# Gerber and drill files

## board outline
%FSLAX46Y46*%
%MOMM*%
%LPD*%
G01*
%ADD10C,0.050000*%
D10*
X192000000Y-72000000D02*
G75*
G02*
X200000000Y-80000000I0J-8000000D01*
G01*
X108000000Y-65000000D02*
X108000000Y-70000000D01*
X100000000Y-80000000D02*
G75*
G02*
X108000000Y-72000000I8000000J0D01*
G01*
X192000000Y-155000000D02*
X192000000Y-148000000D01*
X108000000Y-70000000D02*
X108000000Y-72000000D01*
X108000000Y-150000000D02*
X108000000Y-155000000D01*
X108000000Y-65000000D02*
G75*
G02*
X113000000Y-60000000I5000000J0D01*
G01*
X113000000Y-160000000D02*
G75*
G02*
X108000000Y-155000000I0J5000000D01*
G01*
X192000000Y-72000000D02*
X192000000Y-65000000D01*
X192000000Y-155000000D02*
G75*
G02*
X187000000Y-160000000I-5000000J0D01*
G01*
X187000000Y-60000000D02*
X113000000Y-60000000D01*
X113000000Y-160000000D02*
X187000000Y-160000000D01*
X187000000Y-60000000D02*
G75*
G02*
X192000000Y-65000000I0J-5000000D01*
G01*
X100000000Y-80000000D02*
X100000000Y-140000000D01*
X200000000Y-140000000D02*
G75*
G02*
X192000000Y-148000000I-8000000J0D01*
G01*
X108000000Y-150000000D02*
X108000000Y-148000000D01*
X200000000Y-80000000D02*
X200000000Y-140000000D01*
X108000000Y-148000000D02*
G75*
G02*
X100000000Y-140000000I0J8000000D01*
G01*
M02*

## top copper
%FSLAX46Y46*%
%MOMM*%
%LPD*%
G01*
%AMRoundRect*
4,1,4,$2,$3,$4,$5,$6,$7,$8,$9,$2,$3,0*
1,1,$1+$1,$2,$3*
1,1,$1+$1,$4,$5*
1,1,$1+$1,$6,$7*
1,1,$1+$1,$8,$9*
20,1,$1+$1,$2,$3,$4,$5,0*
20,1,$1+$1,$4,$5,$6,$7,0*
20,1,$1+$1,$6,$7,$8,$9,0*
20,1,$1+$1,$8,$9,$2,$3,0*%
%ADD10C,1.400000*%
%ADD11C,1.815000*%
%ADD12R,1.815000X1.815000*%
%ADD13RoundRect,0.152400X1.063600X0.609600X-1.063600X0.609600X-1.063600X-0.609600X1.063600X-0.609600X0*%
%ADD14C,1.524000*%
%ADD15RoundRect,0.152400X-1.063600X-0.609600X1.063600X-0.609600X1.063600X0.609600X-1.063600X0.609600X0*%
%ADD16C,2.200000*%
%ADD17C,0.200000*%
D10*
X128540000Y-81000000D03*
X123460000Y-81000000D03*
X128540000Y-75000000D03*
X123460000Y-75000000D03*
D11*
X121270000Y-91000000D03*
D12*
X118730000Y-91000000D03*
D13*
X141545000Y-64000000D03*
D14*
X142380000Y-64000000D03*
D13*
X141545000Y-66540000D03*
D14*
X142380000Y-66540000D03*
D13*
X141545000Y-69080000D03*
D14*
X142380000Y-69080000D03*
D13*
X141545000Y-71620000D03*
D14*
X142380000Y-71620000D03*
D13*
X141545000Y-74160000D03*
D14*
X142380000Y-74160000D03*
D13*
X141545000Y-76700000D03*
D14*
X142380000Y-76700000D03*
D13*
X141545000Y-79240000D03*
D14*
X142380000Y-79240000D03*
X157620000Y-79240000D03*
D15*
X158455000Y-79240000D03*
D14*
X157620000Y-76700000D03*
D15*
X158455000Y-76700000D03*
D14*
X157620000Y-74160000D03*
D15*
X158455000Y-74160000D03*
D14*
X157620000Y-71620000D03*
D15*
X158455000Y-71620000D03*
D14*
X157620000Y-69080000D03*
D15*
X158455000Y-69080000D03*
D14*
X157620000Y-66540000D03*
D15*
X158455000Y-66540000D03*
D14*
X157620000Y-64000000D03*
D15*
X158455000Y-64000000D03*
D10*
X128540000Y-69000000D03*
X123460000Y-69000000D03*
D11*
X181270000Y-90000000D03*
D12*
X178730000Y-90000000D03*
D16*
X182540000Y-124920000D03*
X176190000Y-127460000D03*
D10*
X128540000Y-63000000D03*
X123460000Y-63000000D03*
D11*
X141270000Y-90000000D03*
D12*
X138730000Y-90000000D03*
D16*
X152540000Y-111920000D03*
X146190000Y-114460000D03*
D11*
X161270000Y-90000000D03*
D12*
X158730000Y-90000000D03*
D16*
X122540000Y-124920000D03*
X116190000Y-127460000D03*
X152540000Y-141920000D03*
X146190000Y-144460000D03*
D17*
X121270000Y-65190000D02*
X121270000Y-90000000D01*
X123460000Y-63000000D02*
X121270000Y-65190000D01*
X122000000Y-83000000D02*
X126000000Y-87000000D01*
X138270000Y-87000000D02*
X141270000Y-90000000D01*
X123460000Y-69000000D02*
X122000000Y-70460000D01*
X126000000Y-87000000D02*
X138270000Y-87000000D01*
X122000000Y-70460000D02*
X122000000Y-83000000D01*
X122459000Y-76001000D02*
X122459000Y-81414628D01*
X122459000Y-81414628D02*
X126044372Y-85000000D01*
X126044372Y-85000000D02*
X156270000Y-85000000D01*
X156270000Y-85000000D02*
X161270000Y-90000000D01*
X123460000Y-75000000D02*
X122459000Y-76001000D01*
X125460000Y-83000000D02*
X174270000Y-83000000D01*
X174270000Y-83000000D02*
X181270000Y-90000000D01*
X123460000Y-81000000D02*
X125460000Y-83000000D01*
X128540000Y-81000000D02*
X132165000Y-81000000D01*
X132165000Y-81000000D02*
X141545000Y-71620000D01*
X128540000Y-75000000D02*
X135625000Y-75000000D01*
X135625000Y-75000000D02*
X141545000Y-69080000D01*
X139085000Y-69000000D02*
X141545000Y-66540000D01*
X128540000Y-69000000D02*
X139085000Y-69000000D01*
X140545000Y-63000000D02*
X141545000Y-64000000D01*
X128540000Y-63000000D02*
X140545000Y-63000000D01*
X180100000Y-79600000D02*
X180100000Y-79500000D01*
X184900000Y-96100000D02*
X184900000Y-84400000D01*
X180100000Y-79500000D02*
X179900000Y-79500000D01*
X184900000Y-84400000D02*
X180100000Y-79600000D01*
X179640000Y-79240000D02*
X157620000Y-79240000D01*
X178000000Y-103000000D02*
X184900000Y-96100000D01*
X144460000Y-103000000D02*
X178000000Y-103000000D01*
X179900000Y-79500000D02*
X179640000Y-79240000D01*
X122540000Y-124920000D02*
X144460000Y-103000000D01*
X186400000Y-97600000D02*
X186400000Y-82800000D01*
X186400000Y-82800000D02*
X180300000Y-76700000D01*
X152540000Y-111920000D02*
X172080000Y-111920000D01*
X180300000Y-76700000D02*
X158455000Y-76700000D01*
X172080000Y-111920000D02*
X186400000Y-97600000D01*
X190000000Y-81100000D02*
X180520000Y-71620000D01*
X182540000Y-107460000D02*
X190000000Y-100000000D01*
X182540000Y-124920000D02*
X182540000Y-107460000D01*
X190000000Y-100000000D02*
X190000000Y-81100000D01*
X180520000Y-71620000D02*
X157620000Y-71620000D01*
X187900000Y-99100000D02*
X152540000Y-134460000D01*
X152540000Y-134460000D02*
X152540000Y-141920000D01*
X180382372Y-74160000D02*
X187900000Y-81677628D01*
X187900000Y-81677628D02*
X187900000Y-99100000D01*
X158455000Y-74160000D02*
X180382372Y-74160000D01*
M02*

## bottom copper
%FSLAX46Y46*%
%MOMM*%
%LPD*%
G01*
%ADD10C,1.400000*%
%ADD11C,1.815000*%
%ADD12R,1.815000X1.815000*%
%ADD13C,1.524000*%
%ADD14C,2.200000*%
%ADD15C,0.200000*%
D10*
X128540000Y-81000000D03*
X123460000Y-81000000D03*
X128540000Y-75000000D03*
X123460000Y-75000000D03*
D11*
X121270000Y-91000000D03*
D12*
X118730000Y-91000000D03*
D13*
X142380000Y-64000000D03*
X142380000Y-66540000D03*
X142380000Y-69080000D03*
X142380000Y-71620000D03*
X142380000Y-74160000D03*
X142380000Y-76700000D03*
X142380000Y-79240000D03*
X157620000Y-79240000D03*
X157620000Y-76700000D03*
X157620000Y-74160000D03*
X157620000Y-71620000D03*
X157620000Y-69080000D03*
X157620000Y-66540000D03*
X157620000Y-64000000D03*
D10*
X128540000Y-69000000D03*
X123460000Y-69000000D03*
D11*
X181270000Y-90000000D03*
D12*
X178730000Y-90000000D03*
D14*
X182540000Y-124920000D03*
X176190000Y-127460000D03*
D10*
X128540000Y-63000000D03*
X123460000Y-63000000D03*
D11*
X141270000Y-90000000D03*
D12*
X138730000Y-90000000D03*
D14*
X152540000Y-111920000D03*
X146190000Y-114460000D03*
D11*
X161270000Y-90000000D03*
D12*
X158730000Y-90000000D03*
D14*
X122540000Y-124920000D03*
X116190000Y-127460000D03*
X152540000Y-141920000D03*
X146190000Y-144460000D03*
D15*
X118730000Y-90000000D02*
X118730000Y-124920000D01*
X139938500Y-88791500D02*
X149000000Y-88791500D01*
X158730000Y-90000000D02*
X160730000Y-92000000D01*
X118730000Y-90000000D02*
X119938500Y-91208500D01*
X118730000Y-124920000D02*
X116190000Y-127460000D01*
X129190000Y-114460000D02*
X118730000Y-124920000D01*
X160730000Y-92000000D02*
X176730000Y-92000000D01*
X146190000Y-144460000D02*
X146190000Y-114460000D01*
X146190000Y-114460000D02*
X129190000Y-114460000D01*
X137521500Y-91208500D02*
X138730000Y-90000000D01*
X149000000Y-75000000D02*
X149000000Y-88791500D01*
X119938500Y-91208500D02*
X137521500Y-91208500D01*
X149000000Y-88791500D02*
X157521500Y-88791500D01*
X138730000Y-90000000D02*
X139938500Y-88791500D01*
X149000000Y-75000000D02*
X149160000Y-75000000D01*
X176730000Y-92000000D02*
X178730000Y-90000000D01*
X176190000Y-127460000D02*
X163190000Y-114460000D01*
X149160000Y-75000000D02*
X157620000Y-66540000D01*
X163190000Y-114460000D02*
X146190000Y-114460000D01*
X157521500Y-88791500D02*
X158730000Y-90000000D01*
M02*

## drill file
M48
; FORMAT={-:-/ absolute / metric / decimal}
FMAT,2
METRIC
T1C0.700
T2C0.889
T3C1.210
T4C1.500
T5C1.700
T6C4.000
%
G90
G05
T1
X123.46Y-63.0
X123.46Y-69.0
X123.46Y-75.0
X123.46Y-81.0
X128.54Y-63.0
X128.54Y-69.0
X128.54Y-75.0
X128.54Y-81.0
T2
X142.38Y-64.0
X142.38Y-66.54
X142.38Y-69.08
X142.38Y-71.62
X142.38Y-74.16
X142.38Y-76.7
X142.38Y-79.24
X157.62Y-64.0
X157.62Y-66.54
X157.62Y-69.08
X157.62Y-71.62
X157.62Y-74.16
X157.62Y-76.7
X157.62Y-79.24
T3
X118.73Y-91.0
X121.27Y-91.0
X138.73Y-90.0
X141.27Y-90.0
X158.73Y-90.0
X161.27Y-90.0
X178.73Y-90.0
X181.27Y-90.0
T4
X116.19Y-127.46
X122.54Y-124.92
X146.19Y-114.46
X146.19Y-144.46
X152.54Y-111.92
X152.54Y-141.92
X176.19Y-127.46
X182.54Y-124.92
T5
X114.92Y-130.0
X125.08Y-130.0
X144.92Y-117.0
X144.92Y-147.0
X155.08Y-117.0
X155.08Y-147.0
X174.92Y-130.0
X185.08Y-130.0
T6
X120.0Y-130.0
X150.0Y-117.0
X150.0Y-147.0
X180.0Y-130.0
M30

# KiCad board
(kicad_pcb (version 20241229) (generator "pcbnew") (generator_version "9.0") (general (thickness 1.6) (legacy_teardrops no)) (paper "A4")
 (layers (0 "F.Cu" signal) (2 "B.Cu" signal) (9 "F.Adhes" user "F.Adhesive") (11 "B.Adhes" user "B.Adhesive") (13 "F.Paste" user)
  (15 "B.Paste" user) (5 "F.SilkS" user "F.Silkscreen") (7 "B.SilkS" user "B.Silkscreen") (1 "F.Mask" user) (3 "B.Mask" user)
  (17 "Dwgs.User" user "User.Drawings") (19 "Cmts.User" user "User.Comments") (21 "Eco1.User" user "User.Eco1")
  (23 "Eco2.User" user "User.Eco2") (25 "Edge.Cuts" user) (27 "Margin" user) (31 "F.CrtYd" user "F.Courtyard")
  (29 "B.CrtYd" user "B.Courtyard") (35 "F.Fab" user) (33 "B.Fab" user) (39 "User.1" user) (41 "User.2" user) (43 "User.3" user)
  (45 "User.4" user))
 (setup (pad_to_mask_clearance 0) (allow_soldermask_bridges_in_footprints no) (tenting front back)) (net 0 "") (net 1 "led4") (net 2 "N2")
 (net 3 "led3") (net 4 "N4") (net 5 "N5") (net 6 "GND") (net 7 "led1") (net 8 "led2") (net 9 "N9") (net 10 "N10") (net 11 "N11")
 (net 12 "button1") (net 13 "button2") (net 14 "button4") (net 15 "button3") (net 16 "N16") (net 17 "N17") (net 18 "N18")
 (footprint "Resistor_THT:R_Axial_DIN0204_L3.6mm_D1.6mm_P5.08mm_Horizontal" (layer "F.Cu") (at 128.54 81 180)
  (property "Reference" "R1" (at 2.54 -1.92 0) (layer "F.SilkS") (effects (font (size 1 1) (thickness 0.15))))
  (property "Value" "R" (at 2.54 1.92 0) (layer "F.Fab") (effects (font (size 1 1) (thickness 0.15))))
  (pad "1" thru_hole circle (at 0 0 180) (size 1.4 1.4) (drill 0.7) (layers "*.Cu" "*.Mask") (remove_unused_layers no) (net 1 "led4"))
  (pad "2" thru_hole circle (at 5.08 0 180) (size 1.4 1.4) (drill 0.7) (layers "*.Cu" "*.Mask") (remove_unused_layers no) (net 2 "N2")))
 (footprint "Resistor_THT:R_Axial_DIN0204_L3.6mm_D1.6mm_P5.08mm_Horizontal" (layer "F.Cu") (at 128.54 75 180)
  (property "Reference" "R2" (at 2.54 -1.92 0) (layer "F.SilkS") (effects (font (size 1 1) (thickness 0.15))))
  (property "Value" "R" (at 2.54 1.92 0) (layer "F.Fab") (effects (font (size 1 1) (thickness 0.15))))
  (pad "1" thru_hole circle (at 0 0 180) (size 1.4 1.4) (drill 0.7) (layers "*.Cu" "*.Mask") (remove_unused_layers no) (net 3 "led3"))
  (pad "2" thru_hole circle (at 5.08 0 180) (size 1.4 1.4) (drill 0.7) (layers "*.Cu" "*.Mask") (remove_unused_layers no) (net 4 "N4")))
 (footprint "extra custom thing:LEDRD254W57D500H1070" (layer "F.Cu") (at 120 91)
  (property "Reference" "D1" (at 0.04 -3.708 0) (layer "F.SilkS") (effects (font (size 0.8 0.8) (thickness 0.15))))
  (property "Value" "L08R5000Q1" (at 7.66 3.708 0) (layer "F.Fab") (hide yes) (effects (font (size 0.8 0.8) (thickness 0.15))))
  (pad "A" thru_hole circle (at 1.27 0) (size 1.815 1.815) (drill 1.21) (layers "*.Cu" "*.Mask") (remove_unused_layers no) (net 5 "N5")
   (solder_mask_margin 0.102))
  (pad "C" thru_hole rect (at -1.27 0) (size 1.815 1.815) (drill 1.21) (layers "*.Cu" "*.Mask") (remove_unused_layers no) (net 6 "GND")
   (solder_mask_margin 0.102)))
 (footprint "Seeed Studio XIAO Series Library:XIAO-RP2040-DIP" (layer "F.Cu") (at 150 71.62)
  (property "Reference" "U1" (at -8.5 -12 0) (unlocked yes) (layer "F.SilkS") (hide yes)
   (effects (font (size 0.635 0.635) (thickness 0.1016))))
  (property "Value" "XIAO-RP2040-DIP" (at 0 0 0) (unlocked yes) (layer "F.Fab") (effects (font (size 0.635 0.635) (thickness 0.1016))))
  (pad "1" smd roundrect (at -8.455 -7.62 180) (size 2.432 1.524) (layers "F.Cu" "F.Mask") (roundrect_rratio 0.1) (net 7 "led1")
   (thermal_bridge_angle 45))
  (pad "1" thru_hole circle (at -7.62 -7.62 180) (size 1.524 1.524) (drill 0.889) (layers "*.Cu" "*.Mask") (remove_unused_layers no)
   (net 7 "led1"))
  (pad "2" smd roundrect (at -8.455 -5.08 180) (size 2.432 1.524) (layers "F.Cu" "F.Mask") (roundrect_rratio 0.1) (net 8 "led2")
   (thermal_bridge_angle 45))
  (pad "2" thru_hole circle (at -7.62 -5.08 180) (size 1.524 1.524) (drill 0.889) (layers "*.Cu" "*.Mask") (remove_unused_layers no)
   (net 8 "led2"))
  (pad "3" smd roundrect (at -8.455 -2.54 180) (size 2.432 1.524) (layers "F.Cu" "F.Mask") (roundrect_rratio 0.1) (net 3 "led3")
   (thermal_bridge_angle 45))
  (pad "3" thru_hole circle (at -7.62 -2.54 180) (size 1.524 1.524) (drill 0.889) (layers "*.Cu" "*.Mask") (remove_unused_layers no)
   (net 3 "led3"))
  (pad "4" smd roundrect (at -8.455 0 180) (size 2.432 1.524) (layers "F.Cu" "F.Mask") (roundrect_rratio 0.1) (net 1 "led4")
   (thermal_bridge_angle 45))
  (pad "4" thru_hole circle (at -7.62 0 180) (size 1.524 1.524) (drill 0.889) (layers "*.Cu" "*.Mask") (remove_unused_layers no)
   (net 1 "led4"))
  (pad "5" smd roundrect (at -8.455 2.54 180) (size 2.432 1.524) (layers "F.Cu" "F.Mask") (roundrect_rratio 0.1) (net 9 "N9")
   (thermal_bridge_angle 45))
  (pad "5" thru_hole circle (at -7.62 2.54 180) (size 1.524 1.524) (drill 0.889) (layers "*.Cu" "*.Mask") (remove_unused_layers no)
   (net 9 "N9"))
  (pad "6" smd roundrect (at -8.455 5.08 180) (size 2.432 1.524) (layers "F.Cu" "F.Mask") (roundrect_rratio 0.1) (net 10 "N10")
   (thermal_bridge_angle 45))
  (pad "6" thru_hole circle (at -7.62 5.08 180) (size 1.524 1.524) (drill 0.889) (layers "*.Cu" "*.Mask") (remove_unused_layers no)
   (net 10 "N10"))
  (pad "7" smd roundrect (at -8.455 7.62 180) (size 2.432 1.524) (layers "F.Cu" "F.Mask") (roundrect_rratio 0.1) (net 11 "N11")
   (thermal_bridge_angle 45))
  (pad "7" thru_hole circle (at -7.62 7.62 180) (size 1.524 1.524) (drill 0.889) (layers "*.Cu" "*.Mask") (remove_unused_layers no)
   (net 11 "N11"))
  (pad "8" thru_hole circle (at 7.62 7.62) (size 1.524 1.524) (drill 0.889) (layers "*.Cu" "*.Mask") (remove_unused_layers no)
   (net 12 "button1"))
  (pad "8" smd roundrect (at 8.455 7.62) (size 2.432 1.524) (layers "F.Cu" "F.Mask") (roundrect_rratio 0.1) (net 12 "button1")
   (thermal_bridge_angle 45))
  (pad "9" thru_hole circle (at 7.62 5.08) (size 1.524 1.524) (drill 0.889) (layers "*.Cu" "*.Mask") (remove_unused_layers no)
   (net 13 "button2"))
  (pad "9" smd roundrect (at 8.455 5.08) (size 2.432 1.524) (layers "F.Cu" "F.Mask") (roundrect_rratio 0.1) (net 13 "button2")
   (thermal_bridge_angle 45))
  (pad "10" thru_hole circle (at 7.62 2.54) (size 1.524 1.524) (drill 0.889) (layers "*.Cu" "*.Mask") (remove_unused_layers no)
   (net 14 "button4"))
  (pad "10" smd roundrect (at 8.455 2.54) (size 2.432 1.524) (layers "F.Cu" "F.Mask") (roundrect_rratio 0.1) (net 14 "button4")
   (thermal_bridge_angle 45))
  (pad "11" thru_hole circle (at 7.62 0) (size 1.524 1.524) (drill 0.889) (layers "*.Cu" "*.Mask") (remove_unused_layers no)
   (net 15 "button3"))
  (pad "11" smd roundrect (at 8.455 0) (size 2.432 1.524) (layers "F.Cu" "F.Mask") (roundrect_rratio 0.1) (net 15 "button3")
   (thermal_bridge_angle 45))
  (pad "12" thru_hole circle (at 7.62 -2.54) (size 1.524 1.524) (drill 0.889) (layers "*.Cu" "*.Mask") (remove_unused_layers no)
   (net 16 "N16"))
  (pad "12" smd roundrect (at 8.455 -2.54) (size 2.432 1.524) (layers "F.Cu" "F.Mask") (roundrect_rratio 0.1) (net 16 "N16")
   (thermal_bridge_angle 45))
  (pad "13" thru_hole circle (at 7.62 -5.08) (size 1.524 1.524) (drill 0.889) (layers "*.Cu" "*.Mask") (remove_unused_layers no)
   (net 6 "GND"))
  (pad "13" smd roundrect (at 8.455 -5.08) (size 2.432 1.524) (layers "F.Cu" "F.Mask") (roundrect_rratio 0.1) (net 6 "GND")
   (thermal_bridge_angle 45))
  (pad "14" thru_hole circle (at 7.62 -7.62) (size 1.524 1.524) (drill 0.889) (layers "*.Cu" "*.Mask") (remove_unused_layers no)
   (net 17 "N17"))
  (pad "14" smd roundrect (at 8.455 -7.62) (size 2.432 1.524) (layers "F.Cu" "F.Mask") (roundrect_rratio 0.1) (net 17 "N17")
   (thermal_bridge_angle 45)))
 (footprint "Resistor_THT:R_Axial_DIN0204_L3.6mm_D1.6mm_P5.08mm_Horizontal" (layer "F.Cu") (at 128.54 69 180)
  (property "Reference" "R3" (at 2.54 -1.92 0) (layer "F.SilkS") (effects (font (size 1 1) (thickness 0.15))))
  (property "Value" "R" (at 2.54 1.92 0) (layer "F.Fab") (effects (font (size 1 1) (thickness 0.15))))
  (pad "1" thru_hole circle (at 0 0 180) (size 1.4 1.4) (drill 0.7) (layers "*.Cu" "*.Mask") (remove_unused_layers no) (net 8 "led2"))
  (pad "2" thru_hole circle (at 5.08 0 180) (size 1.4 1.4) (drill 0.7) (layers "*.Cu" "*.Mask") (remove_unused_layers no) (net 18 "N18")))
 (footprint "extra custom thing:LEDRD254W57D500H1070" (layer "F.Cu") (at 180 90)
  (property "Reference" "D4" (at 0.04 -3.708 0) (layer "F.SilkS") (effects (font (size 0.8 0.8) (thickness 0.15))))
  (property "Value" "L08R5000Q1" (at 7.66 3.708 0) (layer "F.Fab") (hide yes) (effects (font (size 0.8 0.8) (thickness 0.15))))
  (pad "A" thru_hole circle (at 1.27 0) (size 1.815 1.815) (drill 1.21) (layers "*.Cu" "*.Mask") (remove_unused_layers no) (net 2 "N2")
   (solder_mask_margin 0.102))
  (pad "C" thru_hole rect (at -1.27 0) (size 1.815 1.815) (drill 1.21) (layers "*.Cu" "*.Mask") (remove_unused_layers no) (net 6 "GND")
   (solder_mask_margin 0.102)))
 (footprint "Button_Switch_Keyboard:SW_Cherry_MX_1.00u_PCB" (layer "F.Cu") (at 182.54 124.92)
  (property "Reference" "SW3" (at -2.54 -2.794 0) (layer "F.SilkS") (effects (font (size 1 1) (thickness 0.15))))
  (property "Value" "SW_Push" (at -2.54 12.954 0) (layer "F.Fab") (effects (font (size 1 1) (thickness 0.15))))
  (pad "" np_thru_hole circle (at -7.62 5.08) (size 1.7 1.7) (drill 1.7) (layers "*.Cu" "*.Mask"))
  (pad "" np_thru_hole circle (at -2.54 5.08) (size 4 4) (drill 4) (layers "*.Cu" "*.Mask"))
  (pad "" np_thru_hole circle (at 2.54 5.08) (size 1.7 1.7) (drill 1.7) (layers "*.Cu" "*.Mask"))
  (pad "1" thru_hole circle (at 0 0) (size 2.2 2.2) (drill 1.5) (layers "*.Cu" "*.Mask") (remove_unused_layers no) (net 15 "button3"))
  (pad "2" thru_hole circle (at -6.35 2.54) (size 2.2 2.2) (drill 1.5) (layers "*.Cu" "*.Mask") (remove_unused_layers no) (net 6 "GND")))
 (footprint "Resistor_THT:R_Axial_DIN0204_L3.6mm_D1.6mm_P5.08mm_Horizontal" (layer "F.Cu") (at 128.54 63 180)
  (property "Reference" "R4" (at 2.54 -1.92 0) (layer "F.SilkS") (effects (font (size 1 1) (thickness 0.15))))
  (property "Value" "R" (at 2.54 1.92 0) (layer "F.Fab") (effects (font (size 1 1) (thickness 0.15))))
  (pad "1" thru_hole circle (at 0 0 180) (size 1.4 1.4) (drill 0.7) (layers "*.Cu" "*.Mask") (remove_unused_layers no) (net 7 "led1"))
  (pad "2" thru_hole circle (at 5.08 0 180) (size 1.4 1.4) (drill 0.7) (layers "*.Cu" "*.Mask") (remove_unused_layers no) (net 5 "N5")))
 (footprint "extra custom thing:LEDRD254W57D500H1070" (layer "F.Cu") (at 140 90)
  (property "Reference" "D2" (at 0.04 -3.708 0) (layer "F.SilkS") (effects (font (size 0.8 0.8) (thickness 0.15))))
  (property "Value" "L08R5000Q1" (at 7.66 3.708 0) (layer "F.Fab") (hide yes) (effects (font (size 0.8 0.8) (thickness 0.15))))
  (pad "A" thru_hole circle (at 1.27 0) (size 1.815 1.815) (drill 1.21) (layers "*.Cu" "*.Mask") (remove_unused_layers no) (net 18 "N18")
   (solder_mask_margin 0.102))
  (pad "C" thru_hole rect (at -1.27 0) (size 1.815 1.815) (drill 1.21) (layers "*.Cu" "*.Mask") (remove_unused_layers no) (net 6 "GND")
   (solder_mask_margin 0.102)))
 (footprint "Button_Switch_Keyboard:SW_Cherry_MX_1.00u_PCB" (layer "F.Cu") (at 152.54 111.92)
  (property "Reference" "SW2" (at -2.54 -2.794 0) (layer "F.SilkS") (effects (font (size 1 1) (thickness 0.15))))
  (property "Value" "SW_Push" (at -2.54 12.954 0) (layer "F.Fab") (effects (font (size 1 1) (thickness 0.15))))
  (pad "" np_thru_hole circle (at -7.62 5.08) (size 1.7 1.7) (drill 1.7) (layers "*.Cu" "*.Mask"))
  (pad "" np_thru_hole circle (at -2.54 5.08) (size 4 4) (drill 4) (layers "*.Cu" "*.Mask"))
  (pad "" np_thru_hole circle (at 2.54 5.08) (size 1.7 1.7) (drill 1.7) (layers "*.Cu" "*.Mask"))
  (pad "1" thru_hole circle (at 0 0) (size 2.2 2.2) (drill 1.5) (layers "*.Cu" "*.Mask") (remove_unused_layers no) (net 13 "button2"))
  (pad "2" thru_hole circle (at -6.35 2.54) (size 2.2 2.2) (drill 1.5) (layers "*.Cu" "*.Mask") (remove_unused_layers no) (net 6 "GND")))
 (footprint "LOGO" (layer "F.Cu") (at 129 104)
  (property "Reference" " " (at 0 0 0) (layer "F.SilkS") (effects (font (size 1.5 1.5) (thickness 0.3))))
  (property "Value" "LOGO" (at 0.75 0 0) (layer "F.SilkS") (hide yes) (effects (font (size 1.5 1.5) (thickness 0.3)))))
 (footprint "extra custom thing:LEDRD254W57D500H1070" (layer "F.Cu") (at 160 90)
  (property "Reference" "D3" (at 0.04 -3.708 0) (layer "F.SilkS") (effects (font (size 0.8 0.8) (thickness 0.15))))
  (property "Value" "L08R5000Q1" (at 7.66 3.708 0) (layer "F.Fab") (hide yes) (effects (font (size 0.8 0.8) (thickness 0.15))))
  (pad "A" thru_hole circle (at 1.27 0) (size 1.815 1.815) (drill 1.21) (layers "*.Cu" "*.Mask") (remove_unused_layers no) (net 4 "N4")
   (solder_mask_margin 0.102))
  (pad "C" thru_hole rect (at -1.27 0) (size 1.815 1.815) (drill 1.21) (layers "*.Cu" "*.Mask") (remove_unused_layers no) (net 6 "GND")
   (solder_mask_margin 0.102)))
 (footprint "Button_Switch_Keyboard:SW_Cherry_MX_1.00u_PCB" (layer "F.Cu") (at 122.54 124.92)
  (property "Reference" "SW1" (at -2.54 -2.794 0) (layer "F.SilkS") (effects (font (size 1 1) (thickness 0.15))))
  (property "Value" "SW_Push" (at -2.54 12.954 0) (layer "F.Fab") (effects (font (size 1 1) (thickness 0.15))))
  (pad "" np_thru_hole circle (at -7.62 5.08) (size 1.7 1.7) (drill 1.7) (layers "*.Cu" "*.Mask"))
  (pad "" np_thru_hole circle (at -2.54 5.08) (size 4 4) (drill 4) (layers "*.Cu" "*.Mask"))
  (pad "" np_thru_hole circle (at 2.54 5.08) (size 1.7 1.7) (drill 1.7) (layers "*.Cu" "*.Mask"))
  (pad "1" thru_hole circle (at 0 0) (size 2.2 2.2) (drill 1.5) (layers "*.Cu" "*.Mask") (remove_unused_layers no) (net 12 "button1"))
  (pad "2" thru_hole circle (at -6.35 2.54) (size 2.2 2.2) (drill 1.5) (layers "*.Cu" "*.Mask") (remove_unused_layers no) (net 6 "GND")))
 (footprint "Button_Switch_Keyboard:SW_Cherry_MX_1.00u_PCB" (layer "F.Cu") (at 152.54 141.92)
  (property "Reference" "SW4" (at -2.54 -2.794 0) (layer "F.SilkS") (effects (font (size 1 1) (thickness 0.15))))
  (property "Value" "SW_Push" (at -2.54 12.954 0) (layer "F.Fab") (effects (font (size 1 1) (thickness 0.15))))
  (pad "" np_thru_hole circle (at -7.62 5.08) (size 1.7 1.7) (drill 1.7) (layers "*.Cu" "*.Mask"))
  (pad "" np_thru_hole circle (at -2.54 5.08) (size 4 4) (drill 4) (layers "*.Cu" "*.Mask"))
  (pad "" np_thru_hole circle (at 2.54 5.08) (size 1.7 1.7) (drill 1.7) (layers "*.Cu" "*.Mask"))
  (pad "1" thru_hole circle (at 0 0) (size 2.2 2.2) (drill 1.5) (layers "*.Cu" "*.Mask") (remove_unused_layers no) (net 14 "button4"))
  (pad "2" thru_hole circle (at -6.35 2.54) (size 2.2 2.2) (drill 1.5) (layers "*.Cu" "*.Mask") (remove_unused_layers no) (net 6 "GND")))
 (gr_arc (start 192 72) (mid 197.656854 74.343146) (end 200 80) (stroke (width 0.05) (type default)) (layer "Edge.Cuts"))
 (gr_line (start 108 65) (end 108 70) (stroke (width 0.05) (type default)) (layer "Edge.Cuts"))
 (gr_arc (start 100 80) (mid 102.343146 74.343146) (end 108 72) (stroke (width 0.05) (type default)) (layer "Edge.Cuts"))
 (gr_line (start 192 155) (end 192 148) (stroke (width 0.05) (type default)) (layer "Edge.Cuts"))
 (gr_line (start 108 70) (end 108 72) (stroke (width 0.05) (type default)) (layer "Edge.Cuts"))
 (gr_line (start 108 150) (end 108 155) (stroke (width 0.05) (type default)) (locked yes) (layer "Edge.Cuts"))
 (gr_arc (start 108 65) (mid 109.464466 61.464466) (end 113 60) (stroke (width 0.05) (type default)) (layer "Edge.Cuts"))
 (gr_arc (start 113 160) (mid 109.464466 158.535534) (end 108 155) (stroke (width 0.05) (type default)) (layer "Edge.Cuts"))
 (gr_line (start 192 72) (end 192 65) (stroke (width 0.05) (type default)) (layer "Edge.Cuts"))
 (gr_arc (start 192 155) (mid 190.535534 158.535534) (end 187 160) (stroke (width 0.05) (type default)) (layer "Edge.Cuts"))
 (gr_line (start 187 60) (end 113 60) (stroke (width 0.05) (type default)) (layer "Edge.Cuts"))
 (gr_line (start 113 160) (end 187 160) (stroke (width 0.05) (type default)) (layer "Edge.Cuts"))
 (gr_arc (start 187 60) (mid 190.535534 61.464466) (end 192 65) (stroke (width 0.05) (type default)) (layer "Edge.Cuts"))
 (gr_line (start 100 80) (end 100 140) (stroke (width 0.05) (type default)) (layer "Edge.Cuts"))
 (gr_arc (start 200 140) (mid 197.656854 145.656854) (end 192 148) (stroke (width 0.05) (type default)) (layer "Edge.Cuts"))
 (gr_line (start 108 150) (end 108 148) (stroke (width 0.05) (type default)) (layer "Edge.Cuts"))
 (gr_line (start 200 80) (end 200 140) (stroke (width 0.05) (type default)) (layer "Edge.Cuts"))
 (gr_arc (start 108 148) (mid 102.343146 145.656854) (end 100 140) (stroke (width 0.05) (type default)) (layer "Edge.Cuts"))
 (segment (start 121.27 65.19) (end 121.27 90) (width 0.2) (layer "F.Cu") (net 5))
 (segment (start 123.46 63) (end 121.27 65.19) (width 0.2) (layer "F.Cu") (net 5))
 (segment (start 118.73 90) (end 118.73 124.92) (width 0.2) (layer "B.Cu") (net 6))
 (segment (start 139.9385 88.7915) (end 149 88.7915) (width 0.2) (layer "B.Cu") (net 6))
 (segment (start 158.73 90) (end 160.73 92) (width 0.2) (layer "B.Cu") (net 6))
 (segment (start 118.73 90) (end 119.9385 91.2085) (width 0.2) (layer "B.Cu") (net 6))
 (segment (start 118.73 124.92) (end 116.19 127.46) (width 0.2) (layer "B.Cu") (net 6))
 (segment (start 129.19 114.46) (end 118.73 124.92) (width 0.2) (layer "B.Cu") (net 6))
 (segment (start 160.73 92) (end 176.73 92) (width 0.2) (layer "B.Cu") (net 6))
 (segment (start 146.19 144.46) (end 146.19 114.46) (width 0.2) (layer "B.Cu") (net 6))
 (segment (start 146.19 114.46) (end 129.19 114.46) (width 0.2) (layer "B.Cu") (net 6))
 (segment (start 137.5215 91.2085) (end 138.73 90) (width 0.2) (layer "B.Cu") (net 6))
 (segment (start 149 75) (end 149 88.7915) (width 0.2) (layer "B.Cu") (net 6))
 (segment (start 119.9385 91.2085) (end 137.5215 91.2085) (width 0.2) (layer "B.Cu") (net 6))
 (segment (start 149 88.7915) (end 157.5215 88.7915) (width 0.2) (layer "B.Cu") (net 6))
 (segment (start 138.73 90) (end 139.9385 88.7915) (width 0.2) (layer "B.Cu") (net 6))
 (segment (start 149 75) (end 149.16 75) (width 0.2) (layer "B.Cu") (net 6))
 (segment (start 176.73 92) (end 178.73 90) (width 0.2) (layer "B.Cu") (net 6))
 (segment (start 176.19 127.46) (end 163.19 114.46) (width 0.2) (layer "B.Cu") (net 6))
 (segment (start 149.16 75) (end 157.62 66.54) (width 0.2) (layer "B.Cu") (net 6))
 (segment (start 163.19 114.46) (end 146.19 114.46) (width 0.2) (layer "B.Cu") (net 6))
 (segment (start 157.5215 88.7915) (end 158.73 90) (width 0.2) (layer "B.Cu") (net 6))
 (segment (start 122 83) (end 126 87) (width 0.2) (layer "F.Cu") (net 18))
 (segment (start 138.27 87) (end 141.27 90) (width 0.2) (layer "F.Cu") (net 18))
 (segment (start 123.46 69) (end 122 70.46) (width 0.2) (layer "F.Cu") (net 18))
 (segment (start 126 87) (end 138.27 87) (width 0.2) (layer "F.Cu") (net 18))
 (segment (start 122 70.46) (end 122 83) (width 0.2) (layer "F.Cu") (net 18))
 (segment (start 122.459 76.001) (end 122.459 81.414628) (width 0.2) (layer "F.Cu") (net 4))
 (segment (start 122.459 81.414628) (end 126.044372 85) (width 0.2) (layer "F.Cu") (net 4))
 (segment (start 126.044372 85) (end 156.27 85) (width 0.2) (layer "F.Cu") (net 4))
 (segment (start 156.27 85) (end 161.27 90) (width 0.2) (layer "F.Cu") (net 4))
 (segment (start 123.46 75) (end 122.459 76.001) (width 0.2) (layer "F.Cu") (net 4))
 (segment (start 125.46 83) (end 174.27 83) (width 0.2) (layer "F.Cu") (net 2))
 (segment (start 174.27 83) (end 181.27 90) (width 0.2) (layer "F.Cu") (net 2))
 (segment (start 123.46 81) (end 125.46 83) (width 0.2) (layer "F.Cu") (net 2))
 (segment (start 128.54 81) (end 132.165 81) (width 0.2) (layer "F.Cu") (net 1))
 (segment (start 132.165 81) (end 141.545 71.62) (width 0.2) (layer "F.Cu") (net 1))
 (segment (start 128.54 75) (end 135.625 75) (width 0.2) (layer "F.Cu") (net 3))
 (segment (start 135.625 75) (end 141.545 69.08) (width 0.2) (layer "F.Cu") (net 3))
 (segment (start 139.085 69) (end 141.545 66.54) (width 0.2) (layer "F.Cu") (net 8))
 (segment (start 128.54 69) (end 139.085 69) (width 0.2) (layer "F.Cu") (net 8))
 (segment (start 140.545 63) (end 141.545 64) (width 0.2) (layer "F.Cu") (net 7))
 (segment (start 128.54 63) (end 140.545 63) (width 0.2) (layer "F.Cu") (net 7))
 (segment (start 180.1 79.6) (end 180.1 79.5) (width 0.2) (layer "F.Cu") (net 12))
 (segment (start 184.9 96.1) (end 184.9 84.4) (width 0.2) (layer "F.Cu") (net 12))
 (segment (start 180.1 79.5) (end 179.9 79.5) (width 0.2) (layer "F.Cu") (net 12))
 (segment (start 184.9 84.4) (end 180.1 79.6) (width 0.2) (layer "F.Cu") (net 12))
 (segment (start 179.64 79.24) (end 157.62 79.24) (width 0.2) (layer "F.Cu") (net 12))
 (segment (start 178 103) (end 184.9 96.1) (width 0.2) (layer "F.Cu") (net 12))
 (segment (start 144.46 103) (end 178 103) (width 0.2) (layer "F.Cu") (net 12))
 (segment (start 179.9 79.5) (end 179.64 79.24) (width 0.2) (layer "F.Cu") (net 12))
 (segment (start 122.54 124.92) (end 144.46 103) (width 0.2) (layer "F.Cu") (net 12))
 (segment (start 186.4 97.6) (end 186.4 82.8) (width 0.2) (layer "F.Cu") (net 13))
 (segment (start 186.4 82.8) (end 180.3 76.7) (width 0.2) (layer "F.Cu") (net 13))
 (segment (start 152.54 111.92) (end 172.08 111.92) (width 0.2) (layer "F.Cu") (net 13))
 (segment (start 180.3 76.7) (end 158.455 76.7) (width 0.2) (layer "F.Cu") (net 13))
 (segment (start 172.08 111.92) (end 186.4 97.6) (width 0.2) (layer "F.Cu") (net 13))
 (segment (start 190 81.1) (end 180.52 71.62) (width 0.2) (layer "F.Cu") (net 15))
 (segment (start 182.54 107.46) (end 190 100) (width 0.2) (layer "F.Cu") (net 15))
 (segment (start 182.54 124.92) (end 182.54 107.46) (width 0.2) (layer "F.Cu") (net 15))
 (segment (start 190 100) (end 190 81.1) (width 0.2) (layer "F.Cu") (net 15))
 (segment (start 180.52 71.62) (end 157.62 71.62) (width 0.2) (layer "F.Cu") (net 15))
 (segment (start 187.9 99.1) (end 152.54 134.46) (width 0.2) (layer "F.Cu") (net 14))
 (segment (start 152.54 134.46) (end 152.54 141.92) (width 0.2) (layer "F.Cu") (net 14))
 (segment (start 180.382372 74.16) (end 187.9 81.677628) (width 0.2) (layer "F.Cu") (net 14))
 (segment (start 187.9 81.677628) (end 187.9 99.1) (width 0.2) (layer "F.Cu") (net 14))
 (segment (start 158.455 74.16) (end 180.382372 74.16) (width 0.2) (layer "F.Cu") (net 14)))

